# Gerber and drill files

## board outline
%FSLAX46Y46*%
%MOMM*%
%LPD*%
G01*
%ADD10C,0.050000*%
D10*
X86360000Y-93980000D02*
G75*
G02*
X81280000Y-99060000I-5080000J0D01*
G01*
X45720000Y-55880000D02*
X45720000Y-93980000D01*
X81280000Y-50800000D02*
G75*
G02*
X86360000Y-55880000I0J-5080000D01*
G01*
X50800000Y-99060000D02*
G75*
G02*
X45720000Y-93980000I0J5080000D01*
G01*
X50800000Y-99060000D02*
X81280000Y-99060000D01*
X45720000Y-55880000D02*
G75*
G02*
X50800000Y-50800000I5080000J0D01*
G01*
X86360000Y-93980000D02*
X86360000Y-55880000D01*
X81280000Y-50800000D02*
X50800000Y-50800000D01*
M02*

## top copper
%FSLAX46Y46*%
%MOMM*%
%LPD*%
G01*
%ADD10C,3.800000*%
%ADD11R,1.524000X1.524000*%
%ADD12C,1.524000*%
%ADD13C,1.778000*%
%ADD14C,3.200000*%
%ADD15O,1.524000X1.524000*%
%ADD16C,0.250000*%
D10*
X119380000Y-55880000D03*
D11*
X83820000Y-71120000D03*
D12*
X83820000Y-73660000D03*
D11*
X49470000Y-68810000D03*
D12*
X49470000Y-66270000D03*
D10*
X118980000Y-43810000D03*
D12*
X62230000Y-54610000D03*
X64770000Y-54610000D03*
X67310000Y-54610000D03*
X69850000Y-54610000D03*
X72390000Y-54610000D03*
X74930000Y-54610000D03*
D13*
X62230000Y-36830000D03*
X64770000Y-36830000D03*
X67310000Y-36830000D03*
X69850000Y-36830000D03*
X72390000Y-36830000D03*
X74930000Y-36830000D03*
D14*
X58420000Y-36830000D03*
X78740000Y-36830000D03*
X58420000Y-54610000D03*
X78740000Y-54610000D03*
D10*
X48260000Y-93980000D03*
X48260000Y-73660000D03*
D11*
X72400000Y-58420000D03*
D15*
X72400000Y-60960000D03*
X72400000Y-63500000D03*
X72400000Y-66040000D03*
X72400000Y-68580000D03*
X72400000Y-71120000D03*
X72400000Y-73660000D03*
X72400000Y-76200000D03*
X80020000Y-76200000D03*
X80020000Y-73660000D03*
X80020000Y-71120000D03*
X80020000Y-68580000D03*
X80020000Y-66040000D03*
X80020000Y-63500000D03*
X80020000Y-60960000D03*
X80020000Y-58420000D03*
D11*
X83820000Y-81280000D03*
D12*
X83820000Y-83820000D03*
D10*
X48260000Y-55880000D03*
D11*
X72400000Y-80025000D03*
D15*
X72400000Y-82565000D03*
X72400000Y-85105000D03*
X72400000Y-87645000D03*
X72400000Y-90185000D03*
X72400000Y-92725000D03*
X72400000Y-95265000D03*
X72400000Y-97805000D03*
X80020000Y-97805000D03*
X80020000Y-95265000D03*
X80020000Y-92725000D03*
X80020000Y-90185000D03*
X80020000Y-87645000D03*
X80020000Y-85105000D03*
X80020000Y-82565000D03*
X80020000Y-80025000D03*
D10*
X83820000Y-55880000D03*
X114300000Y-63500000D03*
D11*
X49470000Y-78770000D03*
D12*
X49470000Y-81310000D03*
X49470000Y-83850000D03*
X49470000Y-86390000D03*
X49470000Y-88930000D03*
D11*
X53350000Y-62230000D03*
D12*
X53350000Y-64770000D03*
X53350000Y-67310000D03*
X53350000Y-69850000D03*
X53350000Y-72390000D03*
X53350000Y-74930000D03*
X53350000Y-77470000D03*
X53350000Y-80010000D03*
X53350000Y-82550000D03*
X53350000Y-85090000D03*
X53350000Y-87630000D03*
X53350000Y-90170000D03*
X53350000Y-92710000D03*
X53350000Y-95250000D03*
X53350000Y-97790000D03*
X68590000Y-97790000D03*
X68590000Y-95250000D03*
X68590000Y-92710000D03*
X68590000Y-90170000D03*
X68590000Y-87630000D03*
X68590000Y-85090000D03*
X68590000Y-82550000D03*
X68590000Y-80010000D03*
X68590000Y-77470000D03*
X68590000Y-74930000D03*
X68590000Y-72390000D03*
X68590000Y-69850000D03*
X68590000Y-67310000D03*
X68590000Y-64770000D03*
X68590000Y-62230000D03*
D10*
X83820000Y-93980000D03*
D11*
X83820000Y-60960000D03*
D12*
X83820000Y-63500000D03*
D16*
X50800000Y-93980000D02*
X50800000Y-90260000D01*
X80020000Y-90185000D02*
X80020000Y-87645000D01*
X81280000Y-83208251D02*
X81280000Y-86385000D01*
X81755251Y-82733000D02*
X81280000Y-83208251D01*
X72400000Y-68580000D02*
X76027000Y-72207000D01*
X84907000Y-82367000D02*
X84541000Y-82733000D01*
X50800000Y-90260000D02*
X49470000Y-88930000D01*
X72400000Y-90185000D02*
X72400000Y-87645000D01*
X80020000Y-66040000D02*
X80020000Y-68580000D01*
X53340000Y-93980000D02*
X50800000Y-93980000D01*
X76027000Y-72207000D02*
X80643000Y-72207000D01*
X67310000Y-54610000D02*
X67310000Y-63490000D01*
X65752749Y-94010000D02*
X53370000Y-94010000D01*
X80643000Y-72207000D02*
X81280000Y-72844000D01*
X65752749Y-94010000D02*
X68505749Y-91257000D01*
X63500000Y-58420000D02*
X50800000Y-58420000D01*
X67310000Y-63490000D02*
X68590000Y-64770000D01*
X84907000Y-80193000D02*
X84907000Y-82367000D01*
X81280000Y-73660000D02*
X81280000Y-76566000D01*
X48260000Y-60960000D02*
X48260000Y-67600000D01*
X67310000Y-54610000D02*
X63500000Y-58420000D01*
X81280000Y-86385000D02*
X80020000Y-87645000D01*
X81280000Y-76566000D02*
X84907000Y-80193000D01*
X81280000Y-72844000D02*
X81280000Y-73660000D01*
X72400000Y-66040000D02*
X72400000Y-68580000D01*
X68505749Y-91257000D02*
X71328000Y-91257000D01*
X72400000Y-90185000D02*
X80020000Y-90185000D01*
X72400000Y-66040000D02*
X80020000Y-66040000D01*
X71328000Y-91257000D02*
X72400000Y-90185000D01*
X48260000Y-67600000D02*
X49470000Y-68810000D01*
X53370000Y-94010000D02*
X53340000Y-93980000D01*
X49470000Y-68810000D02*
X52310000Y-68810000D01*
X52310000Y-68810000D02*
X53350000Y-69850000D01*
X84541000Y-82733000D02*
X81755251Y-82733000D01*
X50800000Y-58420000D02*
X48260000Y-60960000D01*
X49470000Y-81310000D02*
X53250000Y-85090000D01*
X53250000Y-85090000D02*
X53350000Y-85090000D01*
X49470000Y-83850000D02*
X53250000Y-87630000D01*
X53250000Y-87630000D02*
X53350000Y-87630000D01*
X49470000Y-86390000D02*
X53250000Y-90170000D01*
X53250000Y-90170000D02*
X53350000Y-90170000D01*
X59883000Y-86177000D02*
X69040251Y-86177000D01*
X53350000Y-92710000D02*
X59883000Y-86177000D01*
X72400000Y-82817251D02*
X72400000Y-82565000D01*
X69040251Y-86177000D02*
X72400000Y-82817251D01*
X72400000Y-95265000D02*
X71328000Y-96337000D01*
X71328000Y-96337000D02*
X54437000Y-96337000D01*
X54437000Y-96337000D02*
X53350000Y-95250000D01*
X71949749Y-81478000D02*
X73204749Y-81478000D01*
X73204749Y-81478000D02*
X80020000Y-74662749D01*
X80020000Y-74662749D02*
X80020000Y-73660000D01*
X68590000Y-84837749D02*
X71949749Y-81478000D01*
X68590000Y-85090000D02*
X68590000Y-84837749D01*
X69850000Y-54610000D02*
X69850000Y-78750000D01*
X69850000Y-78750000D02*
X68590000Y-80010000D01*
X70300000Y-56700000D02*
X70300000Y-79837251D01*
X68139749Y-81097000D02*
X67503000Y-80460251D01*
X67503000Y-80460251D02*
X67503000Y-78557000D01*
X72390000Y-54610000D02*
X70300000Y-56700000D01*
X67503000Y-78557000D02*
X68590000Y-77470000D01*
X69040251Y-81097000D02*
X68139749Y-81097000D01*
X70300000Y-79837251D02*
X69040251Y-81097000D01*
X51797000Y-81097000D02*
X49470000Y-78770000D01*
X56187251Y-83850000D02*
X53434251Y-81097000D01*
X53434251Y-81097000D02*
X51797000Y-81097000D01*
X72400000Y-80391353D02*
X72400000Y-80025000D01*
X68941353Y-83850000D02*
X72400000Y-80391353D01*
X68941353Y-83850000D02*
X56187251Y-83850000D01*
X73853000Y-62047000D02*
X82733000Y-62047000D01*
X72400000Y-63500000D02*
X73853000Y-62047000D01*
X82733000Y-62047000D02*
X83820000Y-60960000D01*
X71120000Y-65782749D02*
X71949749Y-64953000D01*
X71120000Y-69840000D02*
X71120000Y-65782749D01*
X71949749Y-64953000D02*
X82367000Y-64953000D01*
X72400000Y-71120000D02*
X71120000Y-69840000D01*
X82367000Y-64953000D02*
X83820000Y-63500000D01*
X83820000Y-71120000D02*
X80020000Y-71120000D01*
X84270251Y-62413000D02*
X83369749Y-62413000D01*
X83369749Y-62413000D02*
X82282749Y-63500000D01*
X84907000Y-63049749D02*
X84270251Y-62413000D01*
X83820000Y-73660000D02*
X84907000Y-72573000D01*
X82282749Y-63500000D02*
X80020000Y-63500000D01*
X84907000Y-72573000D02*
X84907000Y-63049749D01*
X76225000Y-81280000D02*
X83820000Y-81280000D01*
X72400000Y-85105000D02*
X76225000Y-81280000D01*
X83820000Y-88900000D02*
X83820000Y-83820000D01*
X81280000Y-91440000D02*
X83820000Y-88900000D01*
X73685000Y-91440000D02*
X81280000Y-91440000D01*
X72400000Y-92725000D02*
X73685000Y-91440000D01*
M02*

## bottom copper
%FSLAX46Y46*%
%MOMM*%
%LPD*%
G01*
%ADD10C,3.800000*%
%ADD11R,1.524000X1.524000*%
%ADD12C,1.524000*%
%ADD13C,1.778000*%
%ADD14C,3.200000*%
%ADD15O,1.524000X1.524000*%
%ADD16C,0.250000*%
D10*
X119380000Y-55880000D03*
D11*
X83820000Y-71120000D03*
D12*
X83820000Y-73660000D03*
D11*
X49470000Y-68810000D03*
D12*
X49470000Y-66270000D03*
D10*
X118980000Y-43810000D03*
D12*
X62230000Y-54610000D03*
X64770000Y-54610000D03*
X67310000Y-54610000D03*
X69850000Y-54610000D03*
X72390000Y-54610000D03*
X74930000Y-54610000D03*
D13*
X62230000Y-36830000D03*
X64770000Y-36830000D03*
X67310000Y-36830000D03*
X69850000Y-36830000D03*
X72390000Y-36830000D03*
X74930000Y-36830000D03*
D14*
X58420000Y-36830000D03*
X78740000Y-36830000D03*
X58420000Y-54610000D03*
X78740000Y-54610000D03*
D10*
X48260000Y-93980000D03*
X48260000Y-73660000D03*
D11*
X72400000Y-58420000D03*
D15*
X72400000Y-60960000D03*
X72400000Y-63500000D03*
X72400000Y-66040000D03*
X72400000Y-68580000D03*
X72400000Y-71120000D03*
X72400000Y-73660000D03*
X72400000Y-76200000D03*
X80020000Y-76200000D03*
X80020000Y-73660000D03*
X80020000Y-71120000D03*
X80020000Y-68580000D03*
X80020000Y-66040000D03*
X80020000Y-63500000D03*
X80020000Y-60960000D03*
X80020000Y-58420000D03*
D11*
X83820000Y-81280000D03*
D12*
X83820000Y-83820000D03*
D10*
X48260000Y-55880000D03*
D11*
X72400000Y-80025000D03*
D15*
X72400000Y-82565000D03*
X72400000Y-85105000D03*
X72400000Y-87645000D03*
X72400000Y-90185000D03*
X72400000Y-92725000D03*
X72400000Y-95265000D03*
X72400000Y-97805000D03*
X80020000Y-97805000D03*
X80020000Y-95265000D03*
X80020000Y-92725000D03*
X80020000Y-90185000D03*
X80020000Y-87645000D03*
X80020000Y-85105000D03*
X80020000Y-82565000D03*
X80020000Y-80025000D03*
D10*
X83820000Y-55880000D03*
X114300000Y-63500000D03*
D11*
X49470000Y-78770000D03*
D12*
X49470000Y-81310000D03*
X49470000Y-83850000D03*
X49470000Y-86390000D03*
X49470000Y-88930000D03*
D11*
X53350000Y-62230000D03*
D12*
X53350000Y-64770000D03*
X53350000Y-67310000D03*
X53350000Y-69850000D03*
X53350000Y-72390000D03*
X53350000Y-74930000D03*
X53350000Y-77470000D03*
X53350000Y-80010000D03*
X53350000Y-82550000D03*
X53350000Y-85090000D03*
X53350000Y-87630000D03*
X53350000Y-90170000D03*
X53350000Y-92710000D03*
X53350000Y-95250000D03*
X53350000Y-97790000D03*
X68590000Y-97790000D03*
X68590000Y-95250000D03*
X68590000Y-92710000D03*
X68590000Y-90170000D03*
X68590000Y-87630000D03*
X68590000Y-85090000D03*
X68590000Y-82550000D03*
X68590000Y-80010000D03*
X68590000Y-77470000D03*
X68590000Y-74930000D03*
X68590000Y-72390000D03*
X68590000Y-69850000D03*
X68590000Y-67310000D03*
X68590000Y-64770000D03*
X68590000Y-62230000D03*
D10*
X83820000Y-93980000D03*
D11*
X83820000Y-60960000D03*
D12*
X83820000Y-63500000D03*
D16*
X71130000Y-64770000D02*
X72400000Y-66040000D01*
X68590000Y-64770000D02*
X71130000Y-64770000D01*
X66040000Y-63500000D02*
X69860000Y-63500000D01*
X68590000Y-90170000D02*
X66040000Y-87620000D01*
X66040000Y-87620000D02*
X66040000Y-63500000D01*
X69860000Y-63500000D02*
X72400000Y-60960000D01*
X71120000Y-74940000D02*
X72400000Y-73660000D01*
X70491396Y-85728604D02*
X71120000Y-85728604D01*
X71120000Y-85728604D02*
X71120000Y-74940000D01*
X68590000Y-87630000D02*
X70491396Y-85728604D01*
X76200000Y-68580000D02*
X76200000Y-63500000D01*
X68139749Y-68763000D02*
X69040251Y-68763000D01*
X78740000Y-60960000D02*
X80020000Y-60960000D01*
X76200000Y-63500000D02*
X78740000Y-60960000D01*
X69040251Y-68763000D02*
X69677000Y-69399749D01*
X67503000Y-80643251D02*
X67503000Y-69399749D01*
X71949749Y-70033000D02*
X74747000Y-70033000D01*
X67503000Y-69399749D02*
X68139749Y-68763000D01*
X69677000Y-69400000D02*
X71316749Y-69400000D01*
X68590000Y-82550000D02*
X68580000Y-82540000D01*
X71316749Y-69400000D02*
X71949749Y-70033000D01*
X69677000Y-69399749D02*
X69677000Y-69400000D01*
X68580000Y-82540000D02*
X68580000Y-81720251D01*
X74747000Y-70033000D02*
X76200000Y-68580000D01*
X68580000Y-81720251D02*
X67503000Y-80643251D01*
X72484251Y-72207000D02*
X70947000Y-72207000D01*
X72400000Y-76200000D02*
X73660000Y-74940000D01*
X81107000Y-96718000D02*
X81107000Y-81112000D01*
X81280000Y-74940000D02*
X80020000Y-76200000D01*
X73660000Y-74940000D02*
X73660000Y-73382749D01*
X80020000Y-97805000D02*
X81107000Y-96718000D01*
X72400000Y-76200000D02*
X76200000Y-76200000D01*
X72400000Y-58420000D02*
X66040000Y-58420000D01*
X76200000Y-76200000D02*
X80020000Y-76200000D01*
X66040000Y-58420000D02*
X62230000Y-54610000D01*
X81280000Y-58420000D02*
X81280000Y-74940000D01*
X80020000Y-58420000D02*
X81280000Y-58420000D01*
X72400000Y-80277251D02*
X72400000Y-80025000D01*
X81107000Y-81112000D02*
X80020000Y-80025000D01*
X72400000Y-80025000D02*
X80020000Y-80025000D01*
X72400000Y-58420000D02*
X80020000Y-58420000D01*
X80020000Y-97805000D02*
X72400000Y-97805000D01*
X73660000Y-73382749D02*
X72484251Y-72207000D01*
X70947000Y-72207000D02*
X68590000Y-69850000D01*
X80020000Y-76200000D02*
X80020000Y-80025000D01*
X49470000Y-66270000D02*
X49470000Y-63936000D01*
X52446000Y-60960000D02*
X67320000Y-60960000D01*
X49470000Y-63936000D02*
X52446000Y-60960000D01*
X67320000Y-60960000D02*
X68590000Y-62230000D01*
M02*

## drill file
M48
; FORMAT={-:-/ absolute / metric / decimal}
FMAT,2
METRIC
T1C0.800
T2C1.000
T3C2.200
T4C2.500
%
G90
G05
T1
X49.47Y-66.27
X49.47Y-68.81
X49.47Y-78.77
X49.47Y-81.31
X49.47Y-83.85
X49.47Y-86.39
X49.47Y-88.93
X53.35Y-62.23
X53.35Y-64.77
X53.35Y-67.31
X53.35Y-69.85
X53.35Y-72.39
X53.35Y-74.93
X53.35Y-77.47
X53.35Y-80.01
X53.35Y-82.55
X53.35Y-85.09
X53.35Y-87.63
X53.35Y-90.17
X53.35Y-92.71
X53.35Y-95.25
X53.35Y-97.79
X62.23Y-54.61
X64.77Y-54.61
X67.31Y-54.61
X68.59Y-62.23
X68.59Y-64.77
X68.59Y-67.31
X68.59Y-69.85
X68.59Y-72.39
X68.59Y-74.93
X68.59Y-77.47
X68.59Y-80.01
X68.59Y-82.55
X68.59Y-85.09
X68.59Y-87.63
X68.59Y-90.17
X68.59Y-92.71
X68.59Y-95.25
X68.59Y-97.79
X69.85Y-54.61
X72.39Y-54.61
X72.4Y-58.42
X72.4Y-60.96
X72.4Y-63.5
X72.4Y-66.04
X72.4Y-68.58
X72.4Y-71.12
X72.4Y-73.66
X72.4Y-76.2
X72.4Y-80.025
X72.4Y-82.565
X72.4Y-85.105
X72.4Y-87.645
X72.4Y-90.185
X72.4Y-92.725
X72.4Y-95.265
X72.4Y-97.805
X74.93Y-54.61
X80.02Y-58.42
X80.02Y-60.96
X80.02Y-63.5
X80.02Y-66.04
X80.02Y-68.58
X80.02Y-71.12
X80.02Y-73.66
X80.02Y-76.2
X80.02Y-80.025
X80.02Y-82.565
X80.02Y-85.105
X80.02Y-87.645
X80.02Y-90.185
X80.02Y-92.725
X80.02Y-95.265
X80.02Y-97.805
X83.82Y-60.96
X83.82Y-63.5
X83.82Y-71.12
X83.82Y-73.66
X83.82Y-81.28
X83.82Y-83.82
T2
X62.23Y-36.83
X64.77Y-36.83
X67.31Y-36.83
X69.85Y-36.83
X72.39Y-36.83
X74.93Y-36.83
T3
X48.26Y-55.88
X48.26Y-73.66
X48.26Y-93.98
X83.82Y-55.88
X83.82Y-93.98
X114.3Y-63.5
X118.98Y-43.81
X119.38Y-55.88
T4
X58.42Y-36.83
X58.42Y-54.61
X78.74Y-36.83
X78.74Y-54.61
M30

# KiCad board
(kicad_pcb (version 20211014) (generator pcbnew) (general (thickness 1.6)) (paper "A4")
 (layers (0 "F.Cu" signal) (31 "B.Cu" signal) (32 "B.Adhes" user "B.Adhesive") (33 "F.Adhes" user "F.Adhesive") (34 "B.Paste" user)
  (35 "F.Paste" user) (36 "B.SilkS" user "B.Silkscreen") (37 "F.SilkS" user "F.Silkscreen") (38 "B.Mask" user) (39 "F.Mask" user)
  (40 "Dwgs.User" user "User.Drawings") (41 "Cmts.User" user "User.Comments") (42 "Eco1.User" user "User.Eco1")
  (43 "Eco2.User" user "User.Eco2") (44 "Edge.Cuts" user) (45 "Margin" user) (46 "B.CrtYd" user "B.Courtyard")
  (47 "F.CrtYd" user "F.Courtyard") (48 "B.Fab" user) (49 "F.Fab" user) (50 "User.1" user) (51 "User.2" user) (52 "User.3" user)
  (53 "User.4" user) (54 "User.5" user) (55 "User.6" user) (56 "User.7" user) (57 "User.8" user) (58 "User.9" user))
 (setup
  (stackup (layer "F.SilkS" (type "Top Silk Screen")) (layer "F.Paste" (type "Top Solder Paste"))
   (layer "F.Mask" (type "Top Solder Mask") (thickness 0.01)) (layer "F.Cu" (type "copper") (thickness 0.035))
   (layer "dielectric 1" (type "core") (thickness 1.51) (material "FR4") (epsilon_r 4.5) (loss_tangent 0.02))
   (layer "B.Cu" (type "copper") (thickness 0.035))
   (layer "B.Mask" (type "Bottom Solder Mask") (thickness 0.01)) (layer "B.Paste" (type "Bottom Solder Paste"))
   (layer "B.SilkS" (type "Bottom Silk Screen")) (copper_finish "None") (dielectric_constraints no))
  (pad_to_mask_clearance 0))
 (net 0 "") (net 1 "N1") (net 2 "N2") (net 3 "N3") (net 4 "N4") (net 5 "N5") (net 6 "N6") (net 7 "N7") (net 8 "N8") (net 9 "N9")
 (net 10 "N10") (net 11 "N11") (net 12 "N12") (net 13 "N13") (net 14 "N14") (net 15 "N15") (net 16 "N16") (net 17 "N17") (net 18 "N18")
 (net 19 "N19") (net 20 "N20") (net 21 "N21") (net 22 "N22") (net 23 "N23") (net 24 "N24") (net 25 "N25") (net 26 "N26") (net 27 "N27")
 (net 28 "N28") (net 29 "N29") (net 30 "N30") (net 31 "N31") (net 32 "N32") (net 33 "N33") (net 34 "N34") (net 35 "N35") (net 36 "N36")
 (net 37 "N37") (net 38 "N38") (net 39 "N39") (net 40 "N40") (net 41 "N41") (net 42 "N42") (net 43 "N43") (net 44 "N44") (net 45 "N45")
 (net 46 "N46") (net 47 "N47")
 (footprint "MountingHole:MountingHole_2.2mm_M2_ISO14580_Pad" (layer "F.Cu") (at 119.38 55.88)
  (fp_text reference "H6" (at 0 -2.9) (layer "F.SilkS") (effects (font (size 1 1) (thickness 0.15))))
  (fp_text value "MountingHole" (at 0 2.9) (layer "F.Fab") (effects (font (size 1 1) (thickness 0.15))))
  (pad "1" thru_hole circle (at 0 0) (size 3.8 3.8) (drill 2.2) (layers *.Cu *.Mask)))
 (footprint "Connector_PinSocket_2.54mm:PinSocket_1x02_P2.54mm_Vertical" (layer "F.Cu") (at 83.82 71.12)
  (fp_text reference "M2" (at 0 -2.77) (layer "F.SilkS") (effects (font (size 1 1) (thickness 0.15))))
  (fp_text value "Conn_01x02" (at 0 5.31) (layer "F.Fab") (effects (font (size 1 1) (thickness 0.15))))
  (pad "1" thru_hole rect (at 0 0) (size 1.524 1.524) (drill 0.8) (layers *.Cu *.Mask) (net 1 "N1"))
  (pad "2" thru_hole circle (at 0 2.54) (size 1.524 1.524) (drill 0.8) (layers *.Cu *.Mask) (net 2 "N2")))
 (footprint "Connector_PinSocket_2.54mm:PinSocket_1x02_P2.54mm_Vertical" (layer "F.Cu") (at 49.47 68.81 180)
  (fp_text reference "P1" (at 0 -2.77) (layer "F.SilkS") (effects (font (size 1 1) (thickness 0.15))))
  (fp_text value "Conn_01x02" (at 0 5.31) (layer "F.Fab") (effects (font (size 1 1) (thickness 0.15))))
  (pad "1" thru_hole rect (at 0 0 180) (size 1.524 1.524) (drill 0.8) (layers *.Cu *.Mask) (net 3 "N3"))
  (pad "2" thru_hole circle (at 0 2.54 180) (size 1.524 1.524) (drill 0.8) (layers *.Cu *.Mask) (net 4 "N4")))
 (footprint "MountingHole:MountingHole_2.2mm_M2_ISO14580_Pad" (layer "F.Cu") (at 118.98 43.81)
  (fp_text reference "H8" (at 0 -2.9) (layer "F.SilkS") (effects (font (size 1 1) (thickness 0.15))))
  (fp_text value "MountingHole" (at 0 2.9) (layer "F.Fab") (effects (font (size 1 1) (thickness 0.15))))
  (pad "1" thru_hole circle (at 0 0) (size 3.8 3.8) (drill 2.2) (layers *.Cu *.Mask)))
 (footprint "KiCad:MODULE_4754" (layer "F.Cu") (at 68.58 45.72)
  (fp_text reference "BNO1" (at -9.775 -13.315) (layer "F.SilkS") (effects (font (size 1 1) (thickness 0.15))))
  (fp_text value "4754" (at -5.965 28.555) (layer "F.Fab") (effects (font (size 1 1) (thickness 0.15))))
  (pad "JP1_1" thru_hole circle locked (at -6.35 8.89) (size 1.524 1.524) (drill 0.8) (layers *.Cu *.Mask) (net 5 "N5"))
  (pad "JP1_2" thru_hole circle locked (at -3.81 8.89) (size 1.524 1.524) (drill 0.8) (layers *.Cu *.Mask) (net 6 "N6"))
  (pad "JP1_3" thru_hole circle locked (at -1.27 8.89) (size 1.524 1.524) (drill 0.8) (layers *.Cu *.Mask) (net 3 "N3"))
  (pad "JP1_4" thru_hole circle locked (at 1.27 8.89) (size 1.524 1.524) (drill 0.8) (layers *.Cu *.Mask) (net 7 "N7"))
  (pad "JP1_5" thru_hole circle locked (at 3.81 8.89) (size 1.524 1.524) (drill 0.8) (layers *.Cu *.Mask) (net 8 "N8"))
  (pad "JP1_6" thru_hole circle locked (at 6.35 8.89) (size 1.524 1.524) (drill 0.8) (layers *.Cu *.Mask) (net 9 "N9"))
  (pad "JP2_1" thru_hole circle locked (at -6.35 -8.89) (size 1.778 1.778) (drill 1) (layers *.Cu *.Mask) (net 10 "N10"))
  (pad "JP2_2" thru_hole circle locked (at -3.81 -8.89) (size 1.778 1.778) (drill 1) (layers *.Cu *.Mask) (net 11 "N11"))
  (pad "JP2_3" thru_hole circle locked (at -1.27 -8.89) (size 1.778 1.778) (drill 1) (layers *.Cu *.Mask) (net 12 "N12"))
  (pad "JP2_4" thru_hole circle locked (at 1.27 -8.89) (size 1.778 1.778) (drill 1) (layers *.Cu *.Mask) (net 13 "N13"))
  (pad "JP2_5" thru_hole circle locked (at 3.81 -8.89) (size 1.778 1.778) (drill 1) (layers *.Cu *.Mask) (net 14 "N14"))
  (pad "JP2_6" thru_hole circle locked (at 6.35 -8.89) (size 1.778 1.778) (drill 1) (layers *.Cu *.Mask) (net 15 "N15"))
  (pad "P1" thru_hole circle locked (at -10.16 -8.89) (size 3.2 3.2) (drill 2.5) (layers *.Cu *.Mask))
  (pad "P2" thru_hole circle locked (at 10.16 -8.89) (size 3.2 3.2) (drill 2.5) (layers *.Cu *.Mask))
  (pad "P3" thru_hole circle locked (at -10.16 8.89) (size 3.2 3.2) (drill 2.5) (layers *.Cu *.Mask))
  (pad "P4" thru_hole circle locked (at 10.16 8.89) (size 3.2 3.2) (drill 2.5) (layers *.Cu *.Mask)))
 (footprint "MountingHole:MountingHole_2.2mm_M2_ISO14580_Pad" (layer "F.Cu") (at 48.26 93.98)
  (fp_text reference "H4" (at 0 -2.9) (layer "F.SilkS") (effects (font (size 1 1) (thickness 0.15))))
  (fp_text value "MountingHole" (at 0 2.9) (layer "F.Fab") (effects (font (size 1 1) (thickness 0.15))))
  (pad "1" thru_hole circle (at 0 0) (size 3.8 3.8) (drill 2.2) (layers *.Cu *.Mask)))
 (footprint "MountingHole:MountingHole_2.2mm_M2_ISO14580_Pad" (layer "F.Cu") (at 48.26 73.66)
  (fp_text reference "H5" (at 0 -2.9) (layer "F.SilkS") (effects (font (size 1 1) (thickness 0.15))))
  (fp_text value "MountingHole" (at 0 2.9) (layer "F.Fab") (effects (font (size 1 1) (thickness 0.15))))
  (pad "1" thru_hole circle (at 0 0) (size 3.8 3.8) (drill 2.2) (layers *.Cu *.Mask)))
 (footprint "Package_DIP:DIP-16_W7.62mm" (layer "F.Cu") (at 72.4 58.42)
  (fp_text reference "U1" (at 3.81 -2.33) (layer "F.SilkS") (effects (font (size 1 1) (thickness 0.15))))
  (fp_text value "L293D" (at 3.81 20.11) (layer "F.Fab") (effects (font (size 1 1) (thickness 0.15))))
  (pad "1" thru_hole rect (at 0 0) (size 1.524 1.524) (drill 0.8) (layers *.Cu *.Mask) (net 5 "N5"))
  (pad "2" thru_hole oval (at 0 2.54) (size 1.524 1.524) (drill 0.8) (layers *.Cu *.Mask) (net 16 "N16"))
  (pad "3" thru_hole oval (at 0 5.08) (size 1.524 1.524) (drill 0.8) (layers *.Cu *.Mask) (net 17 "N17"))
  (pad "4" thru_hole oval (at 0 7.62) (size 1.524 1.524) (drill 0.8) (layers *.Cu *.Mask) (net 3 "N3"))
  (pad "5" thru_hole oval (at 0 10.16) (size 1.524 1.524) (drill 0.8) (layers *.Cu *.Mask) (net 3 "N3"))
  (pad "6" thru_hole oval (at 0 12.7) (size 1.524 1.524) (drill 0.8) (layers *.Cu *.Mask) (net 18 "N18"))
  (pad "7" thru_hole oval (at 0 15.24) (size 1.524 1.524) (drill 0.8) (layers *.Cu *.Mask) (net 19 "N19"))
  (pad "8" thru_hole oval (at 0 17.78) (size 1.524 1.524) (drill 0.8) (layers *.Cu *.Mask) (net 5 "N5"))
  (pad "9" thru_hole oval (at 7.62 17.78) (size 1.524 1.524) (drill 0.8) (layers *.Cu *.Mask) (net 5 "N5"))
  (pad "10" thru_hole oval (at 7.62 15.24) (size 1.524 1.524) (drill 0.8) (layers *.Cu *.Mask) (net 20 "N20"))
  (pad "11" thru_hole oval (at 7.62 12.7) (size 1.524 1.524) (drill 0.8) (layers *.Cu *.Mask) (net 1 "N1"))
  (pad "12" thru_hole oval (at 7.62 10.16) (size 1.524 1.524) (drill 0.8) (layers *.Cu *.Mask) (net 3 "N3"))
  (pad "13" thru_hole oval (at 7.62 7.62) (size 1.524 1.524) (drill 0.8) (layers *.Cu *.Mask) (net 3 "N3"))
  (pad "14" thru_hole oval (at 7.62 5.08) (size 1.524 1.524) (drill 0.8) (layers *.Cu *.Mask) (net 2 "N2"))
  (pad "15" thru_hole oval (at 7.62 2.54) (size 1.524 1.524) (drill 0.8) (layers *.Cu *.Mask) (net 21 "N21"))
  (pad "16" thru_hole oval (at 7.62 0) (size 1.524 1.524) (drill 0.8) (layers *.Cu *.Mask) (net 5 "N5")))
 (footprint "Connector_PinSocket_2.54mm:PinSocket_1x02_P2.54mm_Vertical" (layer "F.Cu") (at 83.82 81.28)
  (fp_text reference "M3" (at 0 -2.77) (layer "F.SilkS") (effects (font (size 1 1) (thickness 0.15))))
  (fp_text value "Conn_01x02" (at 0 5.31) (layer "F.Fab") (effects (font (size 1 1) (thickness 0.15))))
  (pad "1" thru_hole rect (at 0 0) (size 1.524 1.524) (drill 0.8) (layers *.Cu *.Mask) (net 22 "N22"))
  (pad "2" thru_hole circle (at 0 2.54) (size 1.524 1.524) (drill 0.8) (layers *.Cu *.Mask) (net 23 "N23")))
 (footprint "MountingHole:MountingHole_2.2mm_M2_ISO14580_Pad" (layer "F.Cu") (at 48.26 55.88)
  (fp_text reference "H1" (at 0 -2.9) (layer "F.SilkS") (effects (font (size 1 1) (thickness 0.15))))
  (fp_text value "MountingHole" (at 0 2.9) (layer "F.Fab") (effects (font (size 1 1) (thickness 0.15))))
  (pad "1" thru_hole circle (at 0 0) (size 3.8 3.8) (drill 2.2) (layers *.Cu *.Mask)))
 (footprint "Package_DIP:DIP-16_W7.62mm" (layer "F.Cu") (at 72.4 80.025)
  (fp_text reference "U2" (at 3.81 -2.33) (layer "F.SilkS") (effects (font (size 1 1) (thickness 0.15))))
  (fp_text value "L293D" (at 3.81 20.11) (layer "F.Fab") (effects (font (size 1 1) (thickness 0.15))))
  (pad "1" thru_hole rect (at 0 0) (size 1.524 1.524) (drill 0.8) (layers *.Cu *.Mask) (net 5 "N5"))
  (pad "2" thru_hole oval (at 0 2.54) (size 1.524 1.524) (drill 0.8) (layers *.Cu *.Mask) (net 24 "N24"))
  (pad "3" thru_hole oval (at 0 5.08) (size 1.524 1.524) (drill 0.8) (layers *.Cu *.Mask) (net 22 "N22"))
  (pad "4" thru_hole oval (at 0 7.62) (size 1.524 1.524) (drill 0.8) (layers *.Cu *.Mask) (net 3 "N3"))
  (pad "5" thru_hole oval (at 0 10.16) (size 1.524 1.524) (drill 0.8) (layers *.Cu *.Mask) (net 3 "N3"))
  (pad "6" thru_hole oval (at 0 12.7) (size 1.524 1.524) (drill 0.8) (layers *.Cu *.Mask) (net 23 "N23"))
  (pad "7" thru_hole oval (at 0 15.24) (size 1.524 1.524) (drill 0.8) (layers *.Cu *.Mask) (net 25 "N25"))
  (pad "8" thru_hole oval (at 0 17.78) (size 1.524 1.524) (drill 0.8) (layers *.Cu *.Mask) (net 5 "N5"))
  (pad "9" thru_hole oval (at 7.62 17.78) (size 1.524 1.524) (drill 0.8) (layers *.Cu *.Mask) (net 5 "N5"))
  (pad "10" thru_hole oval (at 7.62 15.24) (size 1.524 1.524) (drill 0.8) (layers *.Cu *.Mask) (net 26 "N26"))
  (pad "11" thru_hole oval (at 7.62 12.7) (size 1.524 1.524) (drill 0.8) (layers *.Cu *.Mask) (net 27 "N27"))
  (pad "12" thru_hole oval (at 7.62 10.16) (size 1.524 1.524) (drill 0.8) (layers *.Cu *.Mask) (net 3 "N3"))
  (pad "13" thru_hole oval (at 7.62 7.62) (size 1.524 1.524) (drill 0.8) (layers *.Cu *.Mask) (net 3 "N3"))
  (pad "14" thru_hole oval (at 7.62 5.08) (size 1.524 1.524) (drill 0.8) (layers *.Cu *.Mask) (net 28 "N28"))
  (pad "15" thru_hole oval (at 7.62 2.54) (size 1.524 1.524) (drill 0.8) (layers *.Cu *.Mask) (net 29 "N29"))
  (pad "16" thru_hole oval (at 7.62 0) (size 1.524 1.524) (drill 0.8) (layers *.Cu *.Mask) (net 5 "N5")))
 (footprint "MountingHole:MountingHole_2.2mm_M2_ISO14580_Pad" (layer "F.Cu") (at 83.82 55.88)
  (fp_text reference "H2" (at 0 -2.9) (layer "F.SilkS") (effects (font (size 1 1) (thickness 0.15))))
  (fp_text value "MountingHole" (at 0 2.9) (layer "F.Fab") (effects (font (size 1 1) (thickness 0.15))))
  (pad "1" thru_hole circle (at 0 0) (size 3.8 3.8) (drill 2.2) (layers *.Cu *.Mask)))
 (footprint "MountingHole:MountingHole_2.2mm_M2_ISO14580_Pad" (layer "F.Cu") (at 114.3 63.5)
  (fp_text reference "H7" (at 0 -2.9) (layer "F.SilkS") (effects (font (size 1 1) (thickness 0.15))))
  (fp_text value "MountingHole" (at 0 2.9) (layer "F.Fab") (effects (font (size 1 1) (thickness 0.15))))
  (pad "1" thru_hole circle (at 0 0) (size 3.8 3.8) (drill 2.2) (layers *.Cu *.Mask)))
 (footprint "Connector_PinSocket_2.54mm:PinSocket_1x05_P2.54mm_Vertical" (layer "F.Cu") (at 49.47 78.77)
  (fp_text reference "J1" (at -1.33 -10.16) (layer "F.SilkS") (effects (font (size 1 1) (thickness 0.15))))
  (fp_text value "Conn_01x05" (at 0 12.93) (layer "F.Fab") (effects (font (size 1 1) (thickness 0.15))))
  (pad "1" thru_hole rect (at 0 0) (size 1.524 1.524) (drill 0.8) (layers *.Cu *.Mask) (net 5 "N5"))
  (pad "2" thru_hole circle (at 0 2.54) (size 1.524 1.524) (drill 0.8) (layers *.Cu *.Mask) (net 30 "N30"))
  (pad "3" thru_hole circle (at 0 5.08) (size 1.524 1.524) (drill 0.8) (layers *.Cu *.Mask) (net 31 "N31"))
  (pad "4" thru_hole circle (at 0 7.62) (size 1.524 1.524) (drill 0.8) (layers *.Cu *.Mask) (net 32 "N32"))
  (pad "5" thru_hole circle (at 0 10.16) (size 1.524 1.524) (drill 0.8) (layers *.Cu *.Mask) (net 3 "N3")))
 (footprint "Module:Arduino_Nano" (layer "F.Cu") (at 53.35 62.23)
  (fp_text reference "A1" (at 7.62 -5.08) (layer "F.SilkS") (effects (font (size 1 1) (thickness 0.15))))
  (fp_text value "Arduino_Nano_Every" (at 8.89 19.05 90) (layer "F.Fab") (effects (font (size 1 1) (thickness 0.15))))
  (pad "1" thru_hole rect (at 0 0) (size 1.524 1.524) (drill 0.8) (layers *.Cu *.Mask) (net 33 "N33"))
  (pad "2" thru_hole circle (at 0 2.54) (size 1.524 1.524) (drill 0.8) (layers *.Cu *.Mask) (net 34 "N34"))
  (pad "3" thru_hole circle (at 0 5.08) (size 1.524 1.524) (drill 0.8) (layers *.Cu *.Mask) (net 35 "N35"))
  (pad "4" thru_hole circle (at 0 7.62) (size 1.524 1.524) (drill 0.8) (layers *.Cu *.Mask) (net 3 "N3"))
  (pad "5" thru_hole circle (at 0 10.16) (size 1.524 1.524) (drill 0.8) (layers *.Cu *.Mask) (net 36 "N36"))
  (pad "6" thru_hole circle (at 0 12.7) (size 1.524 1.524) (drill 0.8) (layers *.Cu *.Mask) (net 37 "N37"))
  (pad "7" thru_hole circle (at 0 15.24) (size 1.524 1.524) (drill 0.8) (layers *.Cu *.Mask) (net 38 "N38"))
  (pad "8" thru_hole circle (at 0 17.78) (size 1.524 1.524) (drill 0.8) (layers *.Cu *.Mask) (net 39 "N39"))
  (pad "9" thru_hole circle (at 0 20.32) (size 1.524 1.524) (drill 0.8) (layers *.Cu *.Mask) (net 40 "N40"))
  (pad "10" thru_hole circle (at 0 22.86) (size 1.524 1.524) (drill 0.8) (layers *.Cu *.Mask) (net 30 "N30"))
  (pad "11" thru_hole circle (at 0 25.4) (size 1.524 1.524) (drill 0.8) (layers *.Cu *.Mask) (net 31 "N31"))
  (pad "12" thru_hole circle (at 0 27.94) (size 1.524 1.524) (drill 0.8) (layers *.Cu *.Mask) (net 32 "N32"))
  (pad "13" thru_hole circle (at 0 30.48) (size 1.524 1.524) (drill 0.8) (layers *.Cu *.Mask) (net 24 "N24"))
  (pad "14" thru_hole circle (at 0 33.02) (size 1.524 1.524) (drill 0.8) (layers *.Cu *.Mask) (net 25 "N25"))
  (pad "15" thru_hole circle (at 0 35.56) (size 1.524 1.524) (drill 0.8) (layers *.Cu *.Mask) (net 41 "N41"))
  (pad "16" thru_hole circle (at 15.24 35.56) (size 1.524 1.524) (drill 0.8) (layers *.Cu *.Mask) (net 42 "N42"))
  (pad "17" thru_hole circle (at 15.24 33.02) (size 1.524 1.524) (drill 0.8) (layers *.Cu *.Mask) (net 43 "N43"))
  (pad "18" thru_hole circle (at 15.24 30.48) (size 1.524 1.524) (drill 0.8) (layers *.Cu *.Mask) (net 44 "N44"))
  (pad "19" thru_hole circle (at 15.24 27.94) (size 1.524 1.524) (drill 0.8) (layers *.Cu *.Mask) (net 16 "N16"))
  (pad "20" thru_hole circle (at 15.24 25.4) (size 1.524 1.524) (drill 0.8) (layers *.Cu *.Mask) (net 19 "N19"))
  (pad "21" thru_hole circle (at 15.24 22.86) (size 1.524 1.524) (drill 0.8) (layers *.Cu *.Mask) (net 20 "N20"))
  (pad "22" thru_hole circle (at 15.24 20.32) (size 1.524 1.524) (drill 0.8) (layers *.Cu *.Mask) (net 21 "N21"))
  (pad "23" thru_hole circle (at 15.24 17.78) (size 1.524 1.524) (drill 0.8) (layers *.Cu *.Mask) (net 7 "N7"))
  (pad "24" thru_hole circle (at 15.24 15.24) (size 1.524 1.524) (drill 0.8) (layers *.Cu *.Mask) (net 8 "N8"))
  (pad "25" thru_hole circle (at 15.24 12.7) (size 1.524 1.524) (drill 0.8) (layers *.Cu *.Mask) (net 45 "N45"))
  (pad "26" thru_hole circle (at 15.24 10.16) (size 1.524 1.524) (drill 0.8) (layers *.Cu *.Mask) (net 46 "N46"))
  (pad "27" thru_hole circle (at 15.24 7.62) (size 1.524 1.524) (drill 0.8) (layers *.Cu *.Mask) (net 5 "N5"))
  (pad "28" thru_hole circle (at 15.24 5.08) (size 1.524 1.524) (drill 0.8) (layers *.Cu *.Mask) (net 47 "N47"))
  (pad "29" thru_hole circle (at 15.24 2.54) (size 1.524 1.524) (drill 0.8) (layers *.Cu *.Mask) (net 3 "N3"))
  (pad "30" thru_hole circle (at 15.24 0) (size 1.524 1.524) (drill 0.8) (layers *.Cu *.Mask) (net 4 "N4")))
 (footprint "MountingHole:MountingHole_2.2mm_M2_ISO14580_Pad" (layer "F.Cu") (at 83.82 93.98)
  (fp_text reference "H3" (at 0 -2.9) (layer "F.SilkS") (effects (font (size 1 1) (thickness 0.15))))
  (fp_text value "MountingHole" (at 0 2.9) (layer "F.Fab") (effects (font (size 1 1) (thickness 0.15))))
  (pad "1" thru_hole circle (at 0 0) (size 3.8 3.8) (drill 2.2) (layers *.Cu *.Mask)))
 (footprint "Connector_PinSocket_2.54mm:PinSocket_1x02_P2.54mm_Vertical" (layer "F.Cu") (at 83.82 60.96)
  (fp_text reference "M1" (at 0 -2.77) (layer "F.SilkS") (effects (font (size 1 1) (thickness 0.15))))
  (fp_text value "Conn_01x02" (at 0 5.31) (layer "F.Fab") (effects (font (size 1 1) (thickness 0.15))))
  (pad "1" thru_hole rect (at 0 0) (size 1.524 1.524) (drill 0.8) (layers *.Cu *.Mask) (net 17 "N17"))
  (pad "2" thru_hole circle (at 0 2.54) (size 1.524 1.524) (drill 0.8) (layers *.Cu *.Mask) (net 18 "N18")))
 (gr_arc (start 86.36 93.98) (mid 84.872102 97.572102) (end 81.28 99.06) (layer "Edge.Cuts") (width 0.05))
 (gr_line (start 45.72 55.88) (end 45.72 93.98) (layer "Edge.Cuts") (width 0.05))
 (gr_arc (start 81.28 50.8) (mid 84.872102 52.287898) (end 86.36 55.88) (layer "Edge.Cuts") (width 0.05))
 (gr_arc (start 50.8 99.06) (mid 47.207898 97.572102) (end 45.72 93.98) (layer "Edge.Cuts") (width 0.05))
 (gr_line (start 50.8 99.06) (end 81.28 99.06) (layer "Edge.Cuts") (width 0.05))
 (gr_arc (start 45.72 55.88) (mid 47.207898 52.287898) (end 50.8 50.8) (layer "Edge.Cuts") (width 0.05))
 (gr_line (start 86.36 93.98) (end 86.36 55.88) (layer "Edge.Cuts") (width 0.05))
 (gr_line (start 81.28 50.8) (end 50.8 50.8) (layer "Edge.Cuts") (width 0.05))
 (segment (start 50.8 93.98) (end 50.8 90.26) (width 0.25) (layer "F.Cu") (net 3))
 (segment (start 80.02 90.185) (end 80.02 87.645) (width 0.25) (layer "F.Cu") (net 3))
 (segment (start 81.28 83.208251) (end 81.28 86.385) (width 0.25) (layer "F.Cu") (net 3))
 (segment (start 81.755251 82.733) (end 81.28 83.208251) (width 0.25) (layer "F.Cu") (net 3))
 (segment (start 72.4 68.58) (end 76.027 72.207) (width 0.25) (layer "F.Cu") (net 3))
 (segment (start 84.907 82.367) (end 84.541 82.733) (width 0.25) (layer "F.Cu") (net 3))
 (segment (start 50.8 90.26) (end 49.47 88.93) (width 0.25) (layer "F.Cu") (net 3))
 (segment (start 72.4 90.185) (end 72.4 87.645) (width 0.25) (layer "F.Cu") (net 3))
 (segment (start 80.02 66.04) (end 80.02 68.58) (width 0.25) (layer "F.Cu") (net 3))
 (segment (start 53.34 93.98) (end 50.8 93.98) (width 0.25) (layer "F.Cu") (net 3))
 (segment (start 76.027 72.207) (end 80.643 72.207) (width 0.25) (layer "F.Cu") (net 3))
 (segment (start 67.31 54.61) (end 67.31 63.49) (width 0.25) (layer "F.Cu") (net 3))
 (segment (start 65.752749 94.01) (end 53.37 94.01) (width 0.25) (layer "F.Cu") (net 3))
 (segment (start 80.643 72.207) (end 81.28 72.844) (width 0.25) (layer "F.Cu") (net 3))
 (segment (start 65.752749 94.01) (end 68.505749 91.257) (width 0.25) (layer "F.Cu") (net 3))
 (segment (start 63.5 58.42) (end 50.8 58.42) (width 0.25) (layer "F.Cu") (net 3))
 (segment (start 67.31 63.49) (end 68.59 64.77) (width 0.25) (layer "F.Cu") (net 3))
 (segment (start 84.907 80.193) (end 84.907 82.367) (width 0.25) (layer "F.Cu") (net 3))
 (segment (start 81.28 73.66) (end 81.28 76.566) (width 0.25) (layer "F.Cu") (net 3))
 (segment (start 48.26 60.96) (end 48.26 67.6) (width 0.25) (layer "F.Cu") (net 3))
 (segment (start 67.31 54.61) (end 63.5 58.42) (width 0.25) (layer "F.Cu") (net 3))
 (segment (start 81.28 86.385) (end 80.02 87.645) (width 0.25) (layer "F.Cu") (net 3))
 (segment (start 81.28 76.566) (end 84.907 80.193) (width 0.25) (layer "F.Cu") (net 3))
 (segment (start 81.28 72.844) (end 81.28 73.66) (width 0.25) (layer "F.Cu") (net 3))
 (segment (start 72.4 66.04) (end 72.4 68.58) (width 0.25) (layer "F.Cu") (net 3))
 (segment (start 68.505749 91.257) (end 71.328 91.257) (width 0.25) (layer "F.Cu") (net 3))
 (segment (start 72.4 90.185) (end 80.02 90.185) (width 0.25) (layer "F.Cu") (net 3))
 (segment (start 72.4 66.04) (end 80.02 66.04) (width 0.25) (layer "F.Cu") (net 3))
 (segment (start 71.328 91.257) (end 72.4 90.185) (width 0.25) (layer "F.Cu") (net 3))
 (segment (start 48.26 67.6) (end 49.47 68.81) (width 0.25) (layer "F.Cu") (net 3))
 (segment (start 53.37 94.01) (end 53.34 93.98) (width 0.25) (layer "F.Cu") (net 3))
 (segment (start 49.47 68.81) (end 52.31 68.81) (width 0.25) (layer "F.Cu") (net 3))
 (segment (start 52.31 68.81) (end 53.35 69.85) (width 0.25) (layer "F.Cu") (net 3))
 (segment (start 84.541 82.733) (end 81.755251 82.733) (width 0.25) (layer "F.Cu") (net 3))
 (segment (start 50.8 58.42) (end 48.26 60.96) (width 0.25) (layer "F.Cu") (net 3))
 (segment (start 71.13 64.77) (end 72.4 66.04) (width 0.25) (layer "B.Cu") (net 3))
 (segment (start 68.59 64.77) (end 71.13 64.77) (width 0.25) (layer "B.Cu") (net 3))
 (segment (start 49.47 81.31) (end 53.25 85.09) (width 0.25) (layer "F.Cu") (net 30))
 (segment (start 53.25 85.09) (end 53.35 85.09) (width 0.25) (layer "F.Cu") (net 30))
 (segment (start 49.47 83.85) (end 53.25 87.63) (width 0.25) (layer "F.Cu") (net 31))
 (segment (start 53.25 87.63) (end 53.35 87.63) (width 0.25) (layer "F.Cu") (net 31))
 (segment (start 49.47 86.39) (end 53.25 90.17) (width 0.25) (layer "F.Cu") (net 32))
 (segment (start 53.25 90.17) (end 53.35 90.17) (width 0.25) (layer "F.Cu") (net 32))
 (segment (start 59.883 86.177) (end 69.040251 86.177) (width 0.25) (layer "F.Cu") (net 24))
 (segment (start 53.35 92.71) (end 59.883 86.177) (width 0.25) (layer "F.Cu") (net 24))
 (segment (start 72.4 82.817251) (end 72.4 82.565) (width 0.25) (layer "F.Cu") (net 24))
 (segment (start 69.040251 86.177) (end 72.4 82.817251) (width 0.25) (layer "F.Cu") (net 24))
 (segment (start 72.4 95.265) (end 71.328 96.337) (width 0.25) (layer "F.Cu") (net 25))
 (segment (start 71.328 96.337) (end 54.437 96.337) (width 0.25) (layer "F.Cu") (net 25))
 (segment (start 54.437 96.337) (end 53.35 95.25) (width 0.25) (layer "F.Cu") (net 25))
 (segment (start 66.04 63.5) (end 69.86 63.5) (width 0.25) (layer "B.Cu") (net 16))
 (segment (start 68.59 90.17) (end 66.04 87.62) (width 0.25) (layer "B.Cu") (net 16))
 (segment (start 66.04 87.62) (end 66.04 63.5) (width 0.25) (layer "B.Cu") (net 16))
 (segment (start 69.86 63.5) (end 72.4 60.96) (width 0.25) (layer "B.Cu") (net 16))
 (segment (start 71.12 74.94) (end 72.4 73.66) (width 0.25) (layer "B.Cu") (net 19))
 (segment (start 70.491396 85.728604) (end 71.12 85.728604) (width 0.25) (layer "B.Cu") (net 19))
 (segment (start 71.12 85.728604) (end 71.12 74.94) (width 0.25) (layer "B.Cu") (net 19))
 (segment (start 68.59 87.63) (end 70.491396 85.728604) (width 0.25) (layer "B.Cu") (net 19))
 (segment (start 71.949749 81.478) (end 73.204749 81.478) (width 0.25) (layer "F.Cu") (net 20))
 (segment (start 73.204749 81.478) (end 80.02 74.662749) (width 0.25) (layer "F.Cu") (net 20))
 (segment (start 80.02 74.662749) (end 80.02 73.66) (width 0.25) (layer "F.Cu") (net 20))
 (segment (start 68.59 84.837749) (end 71.949749 81.478) (width 0.25) (layer "F.Cu") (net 20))
 (segment (start 68.59 85.09) (end 68.59 84.837749) (width 0.25) (layer "F.Cu") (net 20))
 (segment (start 76.2 68.58) (end 76.2 63.5) (width 0.25) (layer "B.Cu") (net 21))
 (segment (start 68.139749 68.763) (end 69.040251 68.763) (width 0.25) (layer "B.Cu") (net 21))
 (segment (start 78.74 60.96) (end 80.02 60.96) (width 0.25) (layer "B.Cu") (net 21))
 (segment (start 76.2 63.5) (end 78.74 60.96) (width 0.25) (layer "B.Cu") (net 21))
 (segment (start 69.040251 68.763) (end 69.677 69.399749) (width 0.25) (layer "B.Cu") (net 21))
 (segment (start 67.503 80.643251) (end 67.503 69.399749) (width 0.25) (layer "B.Cu") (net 21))
 (segment (start 71.949749 70.033) (end 74.747 70.033) (width 0.25) (layer "B.Cu") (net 21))
 (segment (start 67.503 69.399749) (end 68.139749 68.763) (width 0.25) (layer "B.Cu") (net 21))
 (segment (start 69.677 69.4) (end 71.316749 69.4) (width 0.25) (layer "B.Cu") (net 21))
 (segment (start 68.59 82.55) (end 68.58 82.54) (width 0.25) (layer "B.Cu") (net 21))
 (segment (start 71.316749 69.4) (end 71.949749 70.033) (width 0.25) (layer "B.Cu") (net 21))
 (segment (start 69.677 69.399749) (end 69.677 69.4) (width 0.25) (layer "B.Cu") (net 21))
 (segment (start 68.58 82.54) (end 68.58 81.720251) (width 0.25) (layer "B.Cu") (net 21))
 (segment (start 74.747 70.033) (end 76.2 68.58) (width 0.25) (layer "B.Cu") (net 21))
 (segment (start 68.58 81.720251) (end 67.503 80.643251) (width 0.25) (layer "B.Cu") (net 21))
 (segment (start 69.85 54.61) (end 69.85 78.75) (width 0.25) (layer "F.Cu") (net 7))
 (segment (start 69.85 78.75) (end 68.59 80.01) (width 0.25) (layer "F.Cu") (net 7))
 (segment (start 70.3 56.7) (end 70.3 79.837251) (width 0.25) (layer "F.Cu") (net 8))
 (segment (start 68.139749 81.097) (end 67.503 80.460251) (width 0.25) (layer "F.Cu") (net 8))
 (segment (start 67.503 80.460251) (end 67.503 78.557) (width 0.25) (layer "F.Cu") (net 8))
 (segment (start 72.39 54.61) (end 70.3 56.7) (width 0.25) (layer "F.Cu") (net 8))
 (segment (start 67.503 78.557) (end 68.59 77.47) (width 0.25) (layer "F.Cu") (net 8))
 (segment (start 69.040251 81.097) (end 68.139749 81.097) (width 0.25) (layer "F.Cu") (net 8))
 (segment (start 70.3 79.837251) (end 69.040251 81.097) (width 0.25) (layer "F.Cu") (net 8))
 (segment (start 51.797 81.097) (end 49.47 78.77) (width 0.25) (layer "F.Cu") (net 5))
 (segment (start 56.187251 83.85) (end 53.434251 81.097) (width 0.25) (layer "F.Cu") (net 5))
 (segment (start 53.434251 81.097) (end 51.797 81.097) (width 0.25) (layer "F.Cu") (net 5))
 (segment (start 72.4 80.391353) (end 72.4 80.025) (width 0.25) (layer "F.Cu") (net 5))
 (segment (start 68.941353 83.85) (end 72.4 80.391353) (width 0.25) (layer "F.Cu") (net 5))
 (segment (start 68.941353 83.85) (end 56.187251 83.85) (width 0.25) (layer "F.Cu") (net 5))
 (segment (start 72.484251 72.207) (end 70.947 72.207) (width 0.25) (layer "B.Cu") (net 5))
 (segment (start 72.4 76.2) (end 73.66 74.94) (width 0.25) (layer "B.Cu") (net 5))
 (segment (start 81.107 96.718) (end 81.107 81.112) (width 0.25) (layer "B.Cu") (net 5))
 (segment (start 81.28 74.94) (end 80.02 76.2) (width 0.25) (layer "B.Cu") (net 5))
 (segment (start 73.66 74.94) (end 73.66 73.382749) (width 0.25) (layer "B.Cu") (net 5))
 (segment (start 80.02 97.805) (end 81.107 96.718) (width 0.25) (layer "B.Cu") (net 5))
 (segment (start 72.4 76.2) (end 76.2 76.2) (width 0.25) (layer "B.Cu") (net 5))
 (segment (start 72.4 58.42) (end 66.04 58.42) (width 0.25) (layer "B.Cu") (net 5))
 (segment (start 76.2 76.2) (end 80.02 76.2) (width 0.25) (layer "B.Cu") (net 5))
 (segment (start 66.04 58.42) (end 62.23 54.61) (width 0.25) (layer "B.Cu") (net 5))
 (segment (start 81.28 58.42) (end 81.28 74.94) (width 0.25) (layer "B.Cu") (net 5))
 (segment (start 80.02 58.42) (end 81.28 58.42) (width 0.25) (layer "B.Cu") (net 5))
 (segment (start 72.4 80.277251) (end 72.4 80.025) (width 0.25) (layer "B.Cu") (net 5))
 (segment (start 81.107 81.112) (end 80.02 80.025) (width 0.25) (layer "B.Cu") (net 5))
 (segment (start 72.4 80.025) (end 80.02 80.025) (width 0.25) (layer "B.Cu") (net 5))
 (segment (start 72.4 58.42) (end 80.02 58.42) (width 0.25) (layer "B.Cu") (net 5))
 (segment (start 80.02 97.805) (end 72.4 97.805) (width 0.25) (layer "B.Cu") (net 5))
 (segment (start 73.66 73.382749) (end 72.484251 72.207) (width 0.25) (layer "B.Cu") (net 5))
 (segment (start 70.947 72.207) (end 68.59 69.85) (width 0.25) (layer "B.Cu") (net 5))
 (segment (start 80.02 76.2) (end 80.02 80.025) (width 0.25) (layer "B.Cu") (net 5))
 (segment (start 49.47 66.27) (end 49.47 63.936) (width 0.25) (layer "B.Cu") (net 4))
 (segment (start 52.446 60.96) (end 67.32 60.96) (width 0.25) (layer "B.Cu") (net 4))
 (segment (start 49.47 63.936) (end 52.446 60.96) (width 0.25) (layer "B.Cu") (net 4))
 (segment (start 67.32 60.96) (end 68.59 62.23) (width 0.25) (layer "B.Cu") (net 4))
 (segment (start 73.853 62.047) (end 82.733 62.047) (width 0.25) (layer "F.Cu") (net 17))
 (segment (start 72.4 63.5) (end 73.853 62.047) (width 0.25) (layer "F.Cu") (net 17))
 (segment (start 82.733 62.047) (end 83.82 60.96) (width 0.25) (layer "F.Cu") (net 17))
 (segment (start 71.12 65.782749) (end 71.949749 64.953) (width 0.25) (layer "F.Cu") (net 18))
 (segment (start 71.12 69.84) (end 71.12 65.782749) (width 0.25) (layer "F.Cu") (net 18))
 (segment (start 71.949749 64.953) (end 82.367 64.953) (width 0.25) (layer "F.Cu") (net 18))
 (segment (start 72.4 71.12) (end 71.12 69.84) (width 0.25) (layer "F.Cu") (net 18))
 (segment (start 82.367 64.953) (end 83.82 63.5) (width 0.25) (layer "F.Cu") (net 18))
 (segment (start 83.82 71.12) (end 80.02 71.12) (width 0.25) (layer "F.Cu") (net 1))
 (segment (start 84.270251 62.413) (end 83.369749 62.413) (width 0.25) (layer "F.Cu") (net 2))
 (segment (start 83.369749 62.413) (end 82.282749 63.5) (width 0.25) (layer "F.Cu") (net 2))
 (segment (start 84.907 63.049749) (end 84.270251 62.413) (width 0.25) (layer "F.Cu") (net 2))
 (segment (start 83.82 73.66) (end 84.907 72.573) (width 0.25) (layer "F.Cu") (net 2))
 (segment (start 82.282749 63.5) (end 80.02 63.5) (width 0.25) (layer "F.Cu") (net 2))
 (segment (start 84.907 72.573) (end 84.907 63.049749) (width 0.25) (layer "F.Cu") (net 2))
 (segment (start 76.225 81.28) (end 83.82 81.28) (width 0.25) (layer "F.Cu") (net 22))
 (segment (start 72.4 85.105) (end 76.225 81.28) (width 0.25) (layer "F.Cu") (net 22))
 (segment (start 83.82 88.9) (end 83.82 83.82) (width 0.25) (layer "F.Cu") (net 23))
 (segment (start 81.28 91.44) (end 83.82 88.9) (width 0.25) (layer "F.Cu") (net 23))
 (segment (start 73.685 91.44) (end 81.28 91.44) (width 0.25) (layer "F.Cu") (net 23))
 (segment (start 72.4 92.725) (end 73.685 91.44) (width 0.25) (layer "F.Cu") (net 23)))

